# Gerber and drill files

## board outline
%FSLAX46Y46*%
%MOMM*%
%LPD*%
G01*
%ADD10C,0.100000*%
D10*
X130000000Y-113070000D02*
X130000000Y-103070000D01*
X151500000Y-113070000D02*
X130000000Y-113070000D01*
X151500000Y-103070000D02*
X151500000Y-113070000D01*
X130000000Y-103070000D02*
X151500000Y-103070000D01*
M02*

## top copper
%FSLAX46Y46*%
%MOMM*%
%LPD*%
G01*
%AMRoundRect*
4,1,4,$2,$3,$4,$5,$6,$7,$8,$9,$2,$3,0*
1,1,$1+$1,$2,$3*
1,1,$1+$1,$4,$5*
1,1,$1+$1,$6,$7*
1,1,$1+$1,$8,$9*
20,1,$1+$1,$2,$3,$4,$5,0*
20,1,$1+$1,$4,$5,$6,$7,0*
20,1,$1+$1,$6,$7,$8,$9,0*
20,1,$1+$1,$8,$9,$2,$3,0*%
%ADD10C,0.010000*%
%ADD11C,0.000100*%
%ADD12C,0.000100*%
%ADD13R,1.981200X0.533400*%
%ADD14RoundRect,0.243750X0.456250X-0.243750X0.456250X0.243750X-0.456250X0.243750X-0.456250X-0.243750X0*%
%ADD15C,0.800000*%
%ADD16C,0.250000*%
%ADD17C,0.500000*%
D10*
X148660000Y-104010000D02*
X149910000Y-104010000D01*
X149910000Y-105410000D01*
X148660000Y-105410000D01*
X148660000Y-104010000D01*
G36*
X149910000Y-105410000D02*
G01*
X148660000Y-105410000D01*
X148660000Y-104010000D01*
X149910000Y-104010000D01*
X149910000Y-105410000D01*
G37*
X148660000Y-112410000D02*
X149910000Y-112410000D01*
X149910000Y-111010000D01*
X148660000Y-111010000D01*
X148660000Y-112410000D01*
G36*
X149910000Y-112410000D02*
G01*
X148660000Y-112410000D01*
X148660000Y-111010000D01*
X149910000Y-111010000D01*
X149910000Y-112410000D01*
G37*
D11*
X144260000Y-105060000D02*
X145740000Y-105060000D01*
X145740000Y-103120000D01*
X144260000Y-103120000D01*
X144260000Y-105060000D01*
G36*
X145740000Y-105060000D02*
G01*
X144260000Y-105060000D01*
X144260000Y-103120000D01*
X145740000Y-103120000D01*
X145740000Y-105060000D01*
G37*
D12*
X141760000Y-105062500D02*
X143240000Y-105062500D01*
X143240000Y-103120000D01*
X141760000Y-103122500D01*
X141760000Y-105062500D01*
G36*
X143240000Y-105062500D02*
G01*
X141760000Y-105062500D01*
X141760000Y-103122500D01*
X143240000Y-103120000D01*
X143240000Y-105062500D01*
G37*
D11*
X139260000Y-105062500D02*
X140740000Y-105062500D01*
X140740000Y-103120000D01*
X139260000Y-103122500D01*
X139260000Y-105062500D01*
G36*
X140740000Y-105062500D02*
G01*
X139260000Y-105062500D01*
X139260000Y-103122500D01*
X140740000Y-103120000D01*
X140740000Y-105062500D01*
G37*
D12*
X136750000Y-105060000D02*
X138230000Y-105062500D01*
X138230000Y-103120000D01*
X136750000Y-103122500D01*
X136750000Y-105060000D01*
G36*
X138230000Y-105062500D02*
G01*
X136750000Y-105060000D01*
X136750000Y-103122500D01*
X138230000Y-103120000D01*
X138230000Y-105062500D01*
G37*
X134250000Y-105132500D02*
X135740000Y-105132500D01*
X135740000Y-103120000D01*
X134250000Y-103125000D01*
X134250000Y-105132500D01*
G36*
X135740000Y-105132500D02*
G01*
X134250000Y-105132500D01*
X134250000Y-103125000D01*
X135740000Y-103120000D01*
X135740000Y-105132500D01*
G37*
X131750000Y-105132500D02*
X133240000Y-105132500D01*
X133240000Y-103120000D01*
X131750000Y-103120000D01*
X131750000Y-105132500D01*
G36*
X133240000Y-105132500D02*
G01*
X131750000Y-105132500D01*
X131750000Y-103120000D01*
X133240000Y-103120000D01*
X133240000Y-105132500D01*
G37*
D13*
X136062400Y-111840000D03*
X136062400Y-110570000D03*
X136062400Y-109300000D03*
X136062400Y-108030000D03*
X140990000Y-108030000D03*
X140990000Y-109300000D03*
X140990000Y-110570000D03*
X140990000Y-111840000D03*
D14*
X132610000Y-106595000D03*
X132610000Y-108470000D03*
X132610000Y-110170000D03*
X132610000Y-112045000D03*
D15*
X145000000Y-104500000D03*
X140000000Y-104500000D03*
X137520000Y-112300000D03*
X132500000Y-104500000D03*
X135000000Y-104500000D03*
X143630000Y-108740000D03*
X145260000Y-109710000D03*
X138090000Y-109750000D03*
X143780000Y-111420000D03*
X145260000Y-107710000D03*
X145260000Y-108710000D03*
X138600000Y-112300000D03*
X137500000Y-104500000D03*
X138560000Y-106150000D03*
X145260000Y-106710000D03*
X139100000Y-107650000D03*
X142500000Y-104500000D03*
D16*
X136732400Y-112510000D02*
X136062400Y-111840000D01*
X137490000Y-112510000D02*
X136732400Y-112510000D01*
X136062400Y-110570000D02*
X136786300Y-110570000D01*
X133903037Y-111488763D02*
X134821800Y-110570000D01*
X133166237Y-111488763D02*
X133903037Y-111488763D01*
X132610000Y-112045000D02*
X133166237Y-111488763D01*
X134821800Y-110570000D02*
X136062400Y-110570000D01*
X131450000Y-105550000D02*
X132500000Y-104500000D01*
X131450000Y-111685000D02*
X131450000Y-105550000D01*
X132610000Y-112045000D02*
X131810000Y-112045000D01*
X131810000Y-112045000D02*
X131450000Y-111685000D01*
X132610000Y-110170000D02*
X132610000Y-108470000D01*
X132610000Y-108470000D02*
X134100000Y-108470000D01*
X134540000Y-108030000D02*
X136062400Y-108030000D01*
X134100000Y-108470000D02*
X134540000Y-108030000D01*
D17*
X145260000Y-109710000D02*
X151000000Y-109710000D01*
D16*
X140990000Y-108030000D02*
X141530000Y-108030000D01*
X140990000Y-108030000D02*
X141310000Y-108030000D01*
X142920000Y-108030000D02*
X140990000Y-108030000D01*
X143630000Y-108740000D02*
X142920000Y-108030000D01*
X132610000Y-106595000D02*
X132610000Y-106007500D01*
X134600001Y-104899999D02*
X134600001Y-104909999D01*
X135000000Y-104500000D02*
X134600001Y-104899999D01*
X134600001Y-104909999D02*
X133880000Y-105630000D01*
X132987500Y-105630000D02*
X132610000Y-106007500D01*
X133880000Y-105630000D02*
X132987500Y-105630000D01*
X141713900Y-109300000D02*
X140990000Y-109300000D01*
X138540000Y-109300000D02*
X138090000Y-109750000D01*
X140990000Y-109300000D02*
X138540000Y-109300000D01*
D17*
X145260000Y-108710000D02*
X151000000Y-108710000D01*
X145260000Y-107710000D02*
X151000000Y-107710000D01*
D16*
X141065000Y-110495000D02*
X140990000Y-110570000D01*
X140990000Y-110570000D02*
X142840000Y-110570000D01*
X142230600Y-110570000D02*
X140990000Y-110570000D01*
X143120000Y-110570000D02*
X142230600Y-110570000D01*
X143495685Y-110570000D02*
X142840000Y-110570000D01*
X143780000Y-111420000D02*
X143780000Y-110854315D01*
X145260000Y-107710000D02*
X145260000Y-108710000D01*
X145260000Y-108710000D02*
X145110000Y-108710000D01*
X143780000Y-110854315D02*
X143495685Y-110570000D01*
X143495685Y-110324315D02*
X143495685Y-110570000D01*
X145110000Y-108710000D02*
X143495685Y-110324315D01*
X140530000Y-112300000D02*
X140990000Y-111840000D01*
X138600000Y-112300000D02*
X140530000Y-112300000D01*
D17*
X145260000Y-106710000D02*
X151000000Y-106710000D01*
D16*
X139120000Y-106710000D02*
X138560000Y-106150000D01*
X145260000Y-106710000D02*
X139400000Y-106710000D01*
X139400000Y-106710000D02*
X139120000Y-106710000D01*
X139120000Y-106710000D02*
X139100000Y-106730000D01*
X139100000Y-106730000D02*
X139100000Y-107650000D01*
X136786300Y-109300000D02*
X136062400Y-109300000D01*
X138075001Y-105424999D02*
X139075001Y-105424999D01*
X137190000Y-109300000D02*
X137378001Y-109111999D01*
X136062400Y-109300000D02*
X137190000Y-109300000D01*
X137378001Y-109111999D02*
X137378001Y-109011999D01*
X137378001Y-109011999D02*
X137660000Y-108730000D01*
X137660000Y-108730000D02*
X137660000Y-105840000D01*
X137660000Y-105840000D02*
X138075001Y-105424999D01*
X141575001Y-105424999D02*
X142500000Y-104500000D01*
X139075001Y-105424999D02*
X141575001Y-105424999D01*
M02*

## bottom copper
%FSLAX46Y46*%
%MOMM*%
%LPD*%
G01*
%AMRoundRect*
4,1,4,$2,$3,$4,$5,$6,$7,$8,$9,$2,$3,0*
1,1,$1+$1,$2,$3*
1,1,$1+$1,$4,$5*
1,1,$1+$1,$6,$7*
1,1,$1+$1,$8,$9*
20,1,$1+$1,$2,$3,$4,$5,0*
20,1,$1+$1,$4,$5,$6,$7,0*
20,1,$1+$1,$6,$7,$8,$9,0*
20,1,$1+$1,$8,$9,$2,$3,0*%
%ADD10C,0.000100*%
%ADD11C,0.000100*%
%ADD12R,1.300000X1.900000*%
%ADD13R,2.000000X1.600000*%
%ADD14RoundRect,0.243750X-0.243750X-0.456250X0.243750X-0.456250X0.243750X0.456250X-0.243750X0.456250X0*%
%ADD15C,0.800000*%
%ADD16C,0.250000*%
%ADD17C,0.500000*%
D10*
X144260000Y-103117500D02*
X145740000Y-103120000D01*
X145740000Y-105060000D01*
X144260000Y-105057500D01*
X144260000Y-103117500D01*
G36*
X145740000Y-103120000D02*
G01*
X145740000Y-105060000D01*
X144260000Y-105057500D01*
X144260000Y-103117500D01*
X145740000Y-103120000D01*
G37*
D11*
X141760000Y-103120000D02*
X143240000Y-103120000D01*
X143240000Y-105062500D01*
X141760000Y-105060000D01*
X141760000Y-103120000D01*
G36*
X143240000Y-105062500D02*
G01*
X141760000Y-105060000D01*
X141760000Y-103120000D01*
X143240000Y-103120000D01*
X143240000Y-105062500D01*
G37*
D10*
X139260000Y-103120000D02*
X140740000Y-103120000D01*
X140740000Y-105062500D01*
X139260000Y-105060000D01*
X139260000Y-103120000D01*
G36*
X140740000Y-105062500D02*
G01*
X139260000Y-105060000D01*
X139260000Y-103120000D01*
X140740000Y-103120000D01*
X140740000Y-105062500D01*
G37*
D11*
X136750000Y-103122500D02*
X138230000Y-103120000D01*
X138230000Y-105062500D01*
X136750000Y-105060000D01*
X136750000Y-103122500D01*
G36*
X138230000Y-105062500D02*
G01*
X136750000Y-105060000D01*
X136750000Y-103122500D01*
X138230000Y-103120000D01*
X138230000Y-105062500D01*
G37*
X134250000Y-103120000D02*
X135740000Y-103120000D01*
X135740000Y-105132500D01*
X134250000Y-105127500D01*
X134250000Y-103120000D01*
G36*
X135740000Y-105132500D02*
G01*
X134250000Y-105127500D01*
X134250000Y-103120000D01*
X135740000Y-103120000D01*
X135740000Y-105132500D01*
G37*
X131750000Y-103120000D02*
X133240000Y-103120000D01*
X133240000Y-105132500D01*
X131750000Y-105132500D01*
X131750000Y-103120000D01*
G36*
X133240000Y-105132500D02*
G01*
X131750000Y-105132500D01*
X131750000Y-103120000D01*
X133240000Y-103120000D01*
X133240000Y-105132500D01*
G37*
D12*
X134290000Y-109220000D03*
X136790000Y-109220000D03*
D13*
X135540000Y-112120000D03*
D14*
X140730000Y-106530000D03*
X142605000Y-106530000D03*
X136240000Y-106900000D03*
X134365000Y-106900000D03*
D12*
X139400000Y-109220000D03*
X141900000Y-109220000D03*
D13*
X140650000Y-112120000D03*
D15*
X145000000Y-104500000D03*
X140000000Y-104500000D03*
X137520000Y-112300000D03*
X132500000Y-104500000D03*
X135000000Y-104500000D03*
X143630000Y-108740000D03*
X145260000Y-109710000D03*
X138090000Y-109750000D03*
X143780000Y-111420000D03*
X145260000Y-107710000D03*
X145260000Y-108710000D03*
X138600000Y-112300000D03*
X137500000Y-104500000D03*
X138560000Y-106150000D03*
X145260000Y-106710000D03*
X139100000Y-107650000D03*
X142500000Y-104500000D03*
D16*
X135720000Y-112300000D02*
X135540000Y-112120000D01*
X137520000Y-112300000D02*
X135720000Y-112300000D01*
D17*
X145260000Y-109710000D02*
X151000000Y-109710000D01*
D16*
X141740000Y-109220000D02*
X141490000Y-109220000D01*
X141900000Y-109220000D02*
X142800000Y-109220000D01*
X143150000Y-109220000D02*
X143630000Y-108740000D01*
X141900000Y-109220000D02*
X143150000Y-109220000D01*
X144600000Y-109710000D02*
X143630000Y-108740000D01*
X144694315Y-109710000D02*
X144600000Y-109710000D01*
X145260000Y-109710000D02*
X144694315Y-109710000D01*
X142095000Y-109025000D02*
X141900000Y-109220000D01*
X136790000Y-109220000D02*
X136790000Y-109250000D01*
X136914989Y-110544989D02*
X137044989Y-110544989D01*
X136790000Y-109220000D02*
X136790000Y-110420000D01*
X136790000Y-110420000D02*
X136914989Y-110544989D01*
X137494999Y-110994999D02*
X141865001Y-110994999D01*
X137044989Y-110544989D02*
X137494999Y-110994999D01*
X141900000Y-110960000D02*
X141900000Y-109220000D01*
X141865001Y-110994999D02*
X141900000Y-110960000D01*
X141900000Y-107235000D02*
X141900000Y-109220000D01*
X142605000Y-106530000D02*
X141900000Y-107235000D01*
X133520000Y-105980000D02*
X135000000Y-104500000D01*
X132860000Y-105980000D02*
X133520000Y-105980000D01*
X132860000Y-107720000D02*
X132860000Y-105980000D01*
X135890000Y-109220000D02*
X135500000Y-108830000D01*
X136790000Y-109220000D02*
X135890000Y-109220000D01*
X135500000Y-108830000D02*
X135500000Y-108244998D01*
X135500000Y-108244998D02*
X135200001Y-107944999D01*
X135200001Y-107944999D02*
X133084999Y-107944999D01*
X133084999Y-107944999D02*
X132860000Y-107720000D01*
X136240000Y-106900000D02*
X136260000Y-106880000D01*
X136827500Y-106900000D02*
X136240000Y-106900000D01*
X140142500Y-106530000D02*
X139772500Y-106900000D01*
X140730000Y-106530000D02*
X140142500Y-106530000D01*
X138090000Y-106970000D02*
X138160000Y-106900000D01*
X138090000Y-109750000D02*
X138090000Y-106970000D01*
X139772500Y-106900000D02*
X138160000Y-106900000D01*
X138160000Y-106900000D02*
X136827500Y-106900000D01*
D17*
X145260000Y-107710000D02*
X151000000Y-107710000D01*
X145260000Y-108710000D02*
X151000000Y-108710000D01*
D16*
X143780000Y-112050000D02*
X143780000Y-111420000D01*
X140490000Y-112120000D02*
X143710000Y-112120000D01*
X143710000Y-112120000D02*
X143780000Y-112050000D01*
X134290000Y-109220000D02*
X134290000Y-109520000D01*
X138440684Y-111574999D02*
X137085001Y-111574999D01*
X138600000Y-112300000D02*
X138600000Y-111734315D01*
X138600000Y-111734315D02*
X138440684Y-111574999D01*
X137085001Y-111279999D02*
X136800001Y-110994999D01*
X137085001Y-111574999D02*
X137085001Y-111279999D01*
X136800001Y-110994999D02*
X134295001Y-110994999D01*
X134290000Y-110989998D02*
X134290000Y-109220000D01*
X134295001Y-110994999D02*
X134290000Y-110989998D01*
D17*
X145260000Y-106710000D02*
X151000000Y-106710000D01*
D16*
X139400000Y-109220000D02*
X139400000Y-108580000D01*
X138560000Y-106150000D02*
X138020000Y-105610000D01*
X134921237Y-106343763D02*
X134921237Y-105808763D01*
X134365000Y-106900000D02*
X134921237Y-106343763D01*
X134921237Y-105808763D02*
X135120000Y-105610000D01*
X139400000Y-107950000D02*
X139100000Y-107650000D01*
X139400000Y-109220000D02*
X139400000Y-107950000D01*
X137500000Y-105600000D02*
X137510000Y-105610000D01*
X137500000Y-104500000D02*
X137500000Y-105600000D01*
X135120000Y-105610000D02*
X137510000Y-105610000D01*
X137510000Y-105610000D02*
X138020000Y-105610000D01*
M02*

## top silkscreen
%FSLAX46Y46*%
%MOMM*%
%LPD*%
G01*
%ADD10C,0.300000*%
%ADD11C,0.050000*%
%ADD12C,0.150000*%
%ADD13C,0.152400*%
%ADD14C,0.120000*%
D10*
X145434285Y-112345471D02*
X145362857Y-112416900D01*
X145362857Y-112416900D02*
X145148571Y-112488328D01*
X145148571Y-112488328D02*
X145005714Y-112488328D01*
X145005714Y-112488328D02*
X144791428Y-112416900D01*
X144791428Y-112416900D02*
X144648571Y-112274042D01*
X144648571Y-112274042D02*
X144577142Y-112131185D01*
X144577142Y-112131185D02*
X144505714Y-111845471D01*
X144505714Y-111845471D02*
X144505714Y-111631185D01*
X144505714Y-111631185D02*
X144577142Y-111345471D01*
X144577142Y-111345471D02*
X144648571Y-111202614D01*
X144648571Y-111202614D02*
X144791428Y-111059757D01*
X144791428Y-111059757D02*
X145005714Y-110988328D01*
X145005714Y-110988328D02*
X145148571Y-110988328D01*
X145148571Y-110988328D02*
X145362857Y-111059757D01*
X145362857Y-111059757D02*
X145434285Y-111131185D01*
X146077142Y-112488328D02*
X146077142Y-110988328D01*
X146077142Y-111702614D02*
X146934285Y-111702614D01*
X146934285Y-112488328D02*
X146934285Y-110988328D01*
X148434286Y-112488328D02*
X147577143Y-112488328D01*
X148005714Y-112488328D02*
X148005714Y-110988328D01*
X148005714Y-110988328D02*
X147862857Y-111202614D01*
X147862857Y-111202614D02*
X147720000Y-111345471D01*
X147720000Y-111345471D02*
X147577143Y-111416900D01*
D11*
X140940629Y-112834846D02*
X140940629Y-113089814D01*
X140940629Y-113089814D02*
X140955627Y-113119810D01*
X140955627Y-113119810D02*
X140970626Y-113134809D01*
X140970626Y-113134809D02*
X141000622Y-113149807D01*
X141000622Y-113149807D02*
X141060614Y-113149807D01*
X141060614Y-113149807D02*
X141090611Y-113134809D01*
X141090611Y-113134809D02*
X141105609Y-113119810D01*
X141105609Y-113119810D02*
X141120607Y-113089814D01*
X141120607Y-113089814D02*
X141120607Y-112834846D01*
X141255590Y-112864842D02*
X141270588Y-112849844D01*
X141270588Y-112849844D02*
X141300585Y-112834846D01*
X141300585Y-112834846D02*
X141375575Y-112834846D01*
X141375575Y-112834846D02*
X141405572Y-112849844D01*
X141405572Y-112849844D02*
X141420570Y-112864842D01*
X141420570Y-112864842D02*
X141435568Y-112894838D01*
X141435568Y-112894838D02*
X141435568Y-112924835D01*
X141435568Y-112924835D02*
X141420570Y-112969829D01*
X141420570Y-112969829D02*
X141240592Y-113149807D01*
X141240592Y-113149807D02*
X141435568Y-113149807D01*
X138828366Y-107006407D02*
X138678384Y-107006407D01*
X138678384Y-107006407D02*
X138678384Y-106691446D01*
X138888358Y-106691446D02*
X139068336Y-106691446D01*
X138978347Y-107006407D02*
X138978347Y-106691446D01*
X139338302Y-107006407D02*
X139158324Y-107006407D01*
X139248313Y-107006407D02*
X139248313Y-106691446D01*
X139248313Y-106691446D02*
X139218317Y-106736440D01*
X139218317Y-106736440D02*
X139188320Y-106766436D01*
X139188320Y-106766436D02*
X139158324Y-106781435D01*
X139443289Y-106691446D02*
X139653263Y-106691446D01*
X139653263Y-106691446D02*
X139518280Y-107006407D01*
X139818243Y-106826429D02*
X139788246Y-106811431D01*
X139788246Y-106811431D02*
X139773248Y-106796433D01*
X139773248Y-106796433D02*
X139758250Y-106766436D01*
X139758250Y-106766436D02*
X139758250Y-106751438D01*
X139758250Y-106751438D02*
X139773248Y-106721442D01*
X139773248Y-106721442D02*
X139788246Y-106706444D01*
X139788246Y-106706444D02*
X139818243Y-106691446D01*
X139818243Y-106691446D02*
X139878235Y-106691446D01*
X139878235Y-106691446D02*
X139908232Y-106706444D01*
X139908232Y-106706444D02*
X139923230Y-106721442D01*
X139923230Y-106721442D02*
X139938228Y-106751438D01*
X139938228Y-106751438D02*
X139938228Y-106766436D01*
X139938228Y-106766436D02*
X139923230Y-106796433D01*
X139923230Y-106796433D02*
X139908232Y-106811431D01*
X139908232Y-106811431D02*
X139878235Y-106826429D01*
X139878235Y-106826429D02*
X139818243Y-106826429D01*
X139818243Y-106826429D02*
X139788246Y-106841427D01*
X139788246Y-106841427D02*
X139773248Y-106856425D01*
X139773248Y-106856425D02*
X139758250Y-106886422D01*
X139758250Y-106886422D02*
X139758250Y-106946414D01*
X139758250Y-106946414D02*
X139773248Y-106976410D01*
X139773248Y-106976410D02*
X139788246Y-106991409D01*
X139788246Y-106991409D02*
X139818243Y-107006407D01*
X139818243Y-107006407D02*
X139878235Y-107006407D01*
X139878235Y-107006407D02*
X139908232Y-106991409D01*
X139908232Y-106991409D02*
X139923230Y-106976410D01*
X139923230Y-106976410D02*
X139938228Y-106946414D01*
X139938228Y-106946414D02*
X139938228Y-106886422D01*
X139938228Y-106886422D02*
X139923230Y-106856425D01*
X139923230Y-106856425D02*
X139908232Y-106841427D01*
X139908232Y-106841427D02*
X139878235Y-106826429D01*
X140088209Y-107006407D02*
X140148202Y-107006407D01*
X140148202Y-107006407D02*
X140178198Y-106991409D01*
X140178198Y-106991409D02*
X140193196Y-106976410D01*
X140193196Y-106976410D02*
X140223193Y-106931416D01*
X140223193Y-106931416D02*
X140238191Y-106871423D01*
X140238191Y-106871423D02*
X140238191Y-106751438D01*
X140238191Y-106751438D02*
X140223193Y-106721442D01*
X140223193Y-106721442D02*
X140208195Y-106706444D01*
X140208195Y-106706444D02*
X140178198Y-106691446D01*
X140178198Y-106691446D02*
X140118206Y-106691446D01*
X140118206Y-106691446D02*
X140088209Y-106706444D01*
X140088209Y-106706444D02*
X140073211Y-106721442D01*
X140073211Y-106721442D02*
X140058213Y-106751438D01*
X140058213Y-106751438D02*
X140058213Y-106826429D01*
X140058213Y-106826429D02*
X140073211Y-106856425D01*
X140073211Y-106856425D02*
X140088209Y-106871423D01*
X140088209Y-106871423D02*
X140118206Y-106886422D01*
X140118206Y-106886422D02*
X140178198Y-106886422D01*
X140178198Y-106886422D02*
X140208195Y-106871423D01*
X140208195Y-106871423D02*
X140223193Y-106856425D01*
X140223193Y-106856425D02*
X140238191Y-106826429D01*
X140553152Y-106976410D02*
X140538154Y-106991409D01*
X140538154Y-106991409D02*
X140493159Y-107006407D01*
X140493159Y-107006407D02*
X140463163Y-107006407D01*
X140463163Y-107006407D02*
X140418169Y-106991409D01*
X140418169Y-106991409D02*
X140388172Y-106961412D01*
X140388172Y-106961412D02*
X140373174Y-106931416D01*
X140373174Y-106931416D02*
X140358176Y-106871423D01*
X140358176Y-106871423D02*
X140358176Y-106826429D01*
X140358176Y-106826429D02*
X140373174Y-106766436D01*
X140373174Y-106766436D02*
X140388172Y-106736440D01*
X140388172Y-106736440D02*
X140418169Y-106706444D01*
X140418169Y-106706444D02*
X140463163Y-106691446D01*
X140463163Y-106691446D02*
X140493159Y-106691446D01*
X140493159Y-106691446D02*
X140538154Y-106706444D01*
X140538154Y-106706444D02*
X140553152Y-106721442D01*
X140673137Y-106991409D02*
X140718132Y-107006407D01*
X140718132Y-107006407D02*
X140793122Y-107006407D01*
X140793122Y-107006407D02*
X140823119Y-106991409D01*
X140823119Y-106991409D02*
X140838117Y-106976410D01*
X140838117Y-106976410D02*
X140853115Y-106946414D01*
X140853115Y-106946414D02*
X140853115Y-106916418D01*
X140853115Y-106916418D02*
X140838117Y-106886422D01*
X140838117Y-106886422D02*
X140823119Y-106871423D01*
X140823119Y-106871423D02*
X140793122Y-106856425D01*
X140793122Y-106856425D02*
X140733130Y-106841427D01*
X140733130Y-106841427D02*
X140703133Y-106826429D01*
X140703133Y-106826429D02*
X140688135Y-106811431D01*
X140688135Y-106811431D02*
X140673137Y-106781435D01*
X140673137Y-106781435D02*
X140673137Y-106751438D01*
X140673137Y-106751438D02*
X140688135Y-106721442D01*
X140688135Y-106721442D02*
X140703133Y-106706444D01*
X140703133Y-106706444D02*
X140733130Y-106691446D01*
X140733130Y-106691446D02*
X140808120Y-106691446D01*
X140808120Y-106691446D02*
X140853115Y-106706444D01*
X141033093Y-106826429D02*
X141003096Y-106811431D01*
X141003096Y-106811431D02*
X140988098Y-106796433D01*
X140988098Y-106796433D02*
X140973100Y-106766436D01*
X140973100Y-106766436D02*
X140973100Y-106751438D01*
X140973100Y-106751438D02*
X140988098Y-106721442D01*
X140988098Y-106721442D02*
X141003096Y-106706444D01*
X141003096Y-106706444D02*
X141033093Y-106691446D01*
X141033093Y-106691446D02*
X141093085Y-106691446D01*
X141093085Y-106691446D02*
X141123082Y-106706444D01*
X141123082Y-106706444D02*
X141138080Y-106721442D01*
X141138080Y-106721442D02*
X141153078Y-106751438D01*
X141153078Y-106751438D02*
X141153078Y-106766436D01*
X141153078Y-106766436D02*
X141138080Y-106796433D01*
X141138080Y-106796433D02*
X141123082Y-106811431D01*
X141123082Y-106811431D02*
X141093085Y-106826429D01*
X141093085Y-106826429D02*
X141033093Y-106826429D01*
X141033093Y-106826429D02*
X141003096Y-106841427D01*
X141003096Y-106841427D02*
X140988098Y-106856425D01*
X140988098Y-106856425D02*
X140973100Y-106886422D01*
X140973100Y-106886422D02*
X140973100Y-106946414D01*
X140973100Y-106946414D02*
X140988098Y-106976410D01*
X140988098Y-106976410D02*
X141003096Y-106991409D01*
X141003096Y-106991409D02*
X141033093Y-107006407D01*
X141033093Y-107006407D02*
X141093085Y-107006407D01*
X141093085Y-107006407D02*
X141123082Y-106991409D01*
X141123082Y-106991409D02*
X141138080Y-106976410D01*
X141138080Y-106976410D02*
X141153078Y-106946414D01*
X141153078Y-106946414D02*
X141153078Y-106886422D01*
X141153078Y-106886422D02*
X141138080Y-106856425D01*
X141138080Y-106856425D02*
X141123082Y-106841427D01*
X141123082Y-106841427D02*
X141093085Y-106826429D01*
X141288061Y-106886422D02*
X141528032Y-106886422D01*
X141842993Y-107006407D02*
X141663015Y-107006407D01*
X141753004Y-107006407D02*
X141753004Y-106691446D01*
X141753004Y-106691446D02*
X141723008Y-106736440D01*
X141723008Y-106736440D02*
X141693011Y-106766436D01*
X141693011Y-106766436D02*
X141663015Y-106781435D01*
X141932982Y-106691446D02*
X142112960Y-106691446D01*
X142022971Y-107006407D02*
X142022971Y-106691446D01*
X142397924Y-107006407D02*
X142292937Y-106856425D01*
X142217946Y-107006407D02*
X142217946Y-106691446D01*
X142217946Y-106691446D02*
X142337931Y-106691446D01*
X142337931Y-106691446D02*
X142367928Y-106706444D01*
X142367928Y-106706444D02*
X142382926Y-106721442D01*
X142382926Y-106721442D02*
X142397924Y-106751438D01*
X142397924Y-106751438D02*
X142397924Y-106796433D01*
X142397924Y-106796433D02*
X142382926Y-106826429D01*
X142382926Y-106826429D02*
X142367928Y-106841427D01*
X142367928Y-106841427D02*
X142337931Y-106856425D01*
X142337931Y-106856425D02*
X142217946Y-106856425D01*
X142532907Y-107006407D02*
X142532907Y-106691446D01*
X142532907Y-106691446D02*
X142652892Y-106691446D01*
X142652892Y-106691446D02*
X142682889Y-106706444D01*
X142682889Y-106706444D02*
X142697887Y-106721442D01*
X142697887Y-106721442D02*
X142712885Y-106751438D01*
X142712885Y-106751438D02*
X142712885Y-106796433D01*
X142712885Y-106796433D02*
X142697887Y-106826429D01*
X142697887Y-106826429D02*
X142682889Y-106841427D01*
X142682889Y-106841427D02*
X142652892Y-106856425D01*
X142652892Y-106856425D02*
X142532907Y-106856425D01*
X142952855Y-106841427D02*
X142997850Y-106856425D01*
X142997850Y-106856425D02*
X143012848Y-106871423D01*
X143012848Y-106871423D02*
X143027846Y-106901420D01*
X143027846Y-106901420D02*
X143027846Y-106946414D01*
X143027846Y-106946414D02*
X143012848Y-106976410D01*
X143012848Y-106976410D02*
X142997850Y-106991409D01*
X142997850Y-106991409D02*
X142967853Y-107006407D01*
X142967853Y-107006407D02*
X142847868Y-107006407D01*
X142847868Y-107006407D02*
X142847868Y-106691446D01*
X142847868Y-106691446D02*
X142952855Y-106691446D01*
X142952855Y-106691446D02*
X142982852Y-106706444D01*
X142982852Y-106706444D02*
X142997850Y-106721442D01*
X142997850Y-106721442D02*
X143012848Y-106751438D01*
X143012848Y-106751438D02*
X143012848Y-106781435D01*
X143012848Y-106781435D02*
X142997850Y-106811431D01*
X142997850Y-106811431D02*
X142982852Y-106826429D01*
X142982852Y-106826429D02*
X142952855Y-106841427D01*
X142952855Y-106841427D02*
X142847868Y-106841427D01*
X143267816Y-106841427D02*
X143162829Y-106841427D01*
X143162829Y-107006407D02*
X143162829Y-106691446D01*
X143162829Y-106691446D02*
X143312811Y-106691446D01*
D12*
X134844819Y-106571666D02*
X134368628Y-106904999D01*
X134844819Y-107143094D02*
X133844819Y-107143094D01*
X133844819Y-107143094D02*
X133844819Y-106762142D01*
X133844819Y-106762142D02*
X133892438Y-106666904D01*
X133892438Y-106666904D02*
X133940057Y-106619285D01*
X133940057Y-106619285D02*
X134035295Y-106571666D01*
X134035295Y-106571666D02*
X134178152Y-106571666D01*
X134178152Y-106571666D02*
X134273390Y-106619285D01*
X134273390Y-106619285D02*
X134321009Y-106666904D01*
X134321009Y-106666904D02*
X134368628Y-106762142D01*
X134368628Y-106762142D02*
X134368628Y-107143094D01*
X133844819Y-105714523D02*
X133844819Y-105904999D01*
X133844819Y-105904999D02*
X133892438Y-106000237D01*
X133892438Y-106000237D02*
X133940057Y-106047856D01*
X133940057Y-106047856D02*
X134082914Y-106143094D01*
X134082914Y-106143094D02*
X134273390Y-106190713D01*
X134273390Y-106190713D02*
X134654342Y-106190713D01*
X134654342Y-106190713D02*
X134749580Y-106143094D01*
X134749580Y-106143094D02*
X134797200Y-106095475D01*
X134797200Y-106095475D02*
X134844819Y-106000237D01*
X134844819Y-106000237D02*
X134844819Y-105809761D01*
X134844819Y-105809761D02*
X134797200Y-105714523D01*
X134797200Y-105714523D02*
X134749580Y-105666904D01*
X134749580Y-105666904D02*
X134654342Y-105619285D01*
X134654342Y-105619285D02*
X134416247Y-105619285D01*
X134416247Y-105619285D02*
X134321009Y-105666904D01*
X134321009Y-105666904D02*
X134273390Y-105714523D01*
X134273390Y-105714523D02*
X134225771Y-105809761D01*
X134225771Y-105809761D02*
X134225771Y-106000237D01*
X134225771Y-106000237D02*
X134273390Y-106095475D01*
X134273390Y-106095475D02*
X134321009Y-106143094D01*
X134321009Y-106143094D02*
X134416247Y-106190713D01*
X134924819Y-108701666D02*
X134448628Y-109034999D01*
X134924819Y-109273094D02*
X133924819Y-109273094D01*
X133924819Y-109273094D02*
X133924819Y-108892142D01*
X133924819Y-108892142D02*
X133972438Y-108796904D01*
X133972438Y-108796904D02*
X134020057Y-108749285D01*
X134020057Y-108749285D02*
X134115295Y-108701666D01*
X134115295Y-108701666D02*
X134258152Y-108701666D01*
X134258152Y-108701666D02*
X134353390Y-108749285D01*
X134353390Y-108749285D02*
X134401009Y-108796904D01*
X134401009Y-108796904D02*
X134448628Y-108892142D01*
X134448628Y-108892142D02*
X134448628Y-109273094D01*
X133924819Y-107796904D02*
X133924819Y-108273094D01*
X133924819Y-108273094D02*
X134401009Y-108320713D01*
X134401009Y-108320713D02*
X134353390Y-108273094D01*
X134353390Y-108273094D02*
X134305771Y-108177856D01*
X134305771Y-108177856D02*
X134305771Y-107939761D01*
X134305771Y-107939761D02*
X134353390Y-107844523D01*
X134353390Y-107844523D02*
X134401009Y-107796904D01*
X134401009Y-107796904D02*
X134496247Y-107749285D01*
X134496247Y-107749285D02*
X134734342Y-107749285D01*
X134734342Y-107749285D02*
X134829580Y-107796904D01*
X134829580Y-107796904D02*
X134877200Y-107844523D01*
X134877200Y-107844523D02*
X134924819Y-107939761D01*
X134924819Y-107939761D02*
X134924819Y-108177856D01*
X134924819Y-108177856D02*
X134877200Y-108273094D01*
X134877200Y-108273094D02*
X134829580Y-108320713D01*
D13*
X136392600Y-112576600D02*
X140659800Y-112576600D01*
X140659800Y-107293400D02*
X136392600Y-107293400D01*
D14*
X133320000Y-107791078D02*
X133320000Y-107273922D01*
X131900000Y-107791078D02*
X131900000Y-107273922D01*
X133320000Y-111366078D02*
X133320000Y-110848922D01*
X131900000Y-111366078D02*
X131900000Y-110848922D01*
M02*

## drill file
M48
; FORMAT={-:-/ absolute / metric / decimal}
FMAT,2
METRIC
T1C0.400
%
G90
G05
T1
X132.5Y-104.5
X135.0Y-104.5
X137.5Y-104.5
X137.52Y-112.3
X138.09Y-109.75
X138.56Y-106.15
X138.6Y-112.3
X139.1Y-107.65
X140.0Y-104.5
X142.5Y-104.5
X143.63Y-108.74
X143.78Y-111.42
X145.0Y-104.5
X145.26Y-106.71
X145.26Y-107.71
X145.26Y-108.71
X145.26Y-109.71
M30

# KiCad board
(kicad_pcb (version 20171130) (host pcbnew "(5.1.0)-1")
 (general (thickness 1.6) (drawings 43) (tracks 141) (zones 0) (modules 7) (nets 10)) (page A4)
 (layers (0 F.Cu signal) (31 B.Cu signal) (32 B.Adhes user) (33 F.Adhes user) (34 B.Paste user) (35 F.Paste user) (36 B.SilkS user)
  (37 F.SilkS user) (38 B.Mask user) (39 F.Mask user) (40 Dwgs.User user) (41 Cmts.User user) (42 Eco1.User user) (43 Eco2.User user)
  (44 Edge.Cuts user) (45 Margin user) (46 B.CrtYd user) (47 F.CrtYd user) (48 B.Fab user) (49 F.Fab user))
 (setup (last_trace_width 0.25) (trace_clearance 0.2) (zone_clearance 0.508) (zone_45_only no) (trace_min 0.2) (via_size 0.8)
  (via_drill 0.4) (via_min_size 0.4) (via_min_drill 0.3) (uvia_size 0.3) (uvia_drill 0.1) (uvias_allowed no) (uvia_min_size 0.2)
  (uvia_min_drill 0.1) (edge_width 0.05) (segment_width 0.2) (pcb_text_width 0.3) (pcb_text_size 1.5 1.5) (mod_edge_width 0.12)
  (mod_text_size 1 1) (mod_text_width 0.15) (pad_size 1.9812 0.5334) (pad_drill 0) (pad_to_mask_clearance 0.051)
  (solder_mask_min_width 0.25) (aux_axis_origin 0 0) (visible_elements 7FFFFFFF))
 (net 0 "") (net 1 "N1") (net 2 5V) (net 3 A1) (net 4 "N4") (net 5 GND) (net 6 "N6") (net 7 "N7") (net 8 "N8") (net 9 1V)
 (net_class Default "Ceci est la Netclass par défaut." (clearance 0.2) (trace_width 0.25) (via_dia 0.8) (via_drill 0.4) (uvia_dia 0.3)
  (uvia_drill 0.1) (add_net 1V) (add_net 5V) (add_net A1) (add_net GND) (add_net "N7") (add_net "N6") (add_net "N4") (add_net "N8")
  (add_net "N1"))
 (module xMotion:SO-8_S (layer F.Cu) (at 138.5262 109.935 180)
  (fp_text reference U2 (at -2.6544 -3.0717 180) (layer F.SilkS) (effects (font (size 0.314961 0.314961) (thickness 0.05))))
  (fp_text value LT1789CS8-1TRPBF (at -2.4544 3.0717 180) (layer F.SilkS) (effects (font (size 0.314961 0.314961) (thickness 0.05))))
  (fp_line (start 2.1336 -2.6416) (end -2.1336 -2.6416) (layer F.SilkS) (width 0.1524))
  (fp_line (start -2.1336 2.6416) (end 2.1336 2.6416) (layer F.SilkS) (width 0.1524))
  (pad 8 smd rect (at 2.4638 -1.905 180) (size 1.9812 0.5334) (layers F.Cu F.Paste F.Mask) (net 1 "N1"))
  (pad 7 smd rect (at 2.4638 -0.635 180) (size 1.9812 0.5334) (layers F.Cu F.Paste F.Mask) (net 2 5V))
  (pad 6 smd rect (at 2.4638 0.635 180) (size 1.9812 0.5334) (layers F.Cu F.Paste F.Mask) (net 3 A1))
  (pad 5 smd rect (at 2.4638 1.905 180) (size 1.9812 0.5334) (layers F.Cu F.Paste F.Mask) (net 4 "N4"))
  (pad 4 smd rect (at -2.4638 1.905 180) (size 1.9812 0.5334) (layers F.Cu F.Paste F.Mask) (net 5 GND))
  (pad 3 smd rect (at -2.4638 0.635 180) (size 1.9812 0.5334) (layers F.Cu F.Paste F.Mask) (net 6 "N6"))
  (pad 2 smd rect (at -2.4638 -0.635 180) (size 1.9812 0.5334) (layers F.Cu F.Paste F.Mask) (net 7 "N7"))
  (pad 1 smd rect (at -2.4638 -1.905 180) (size 1.9812 0.5334) (layers F.Cu F.Paste F.Mask) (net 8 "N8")))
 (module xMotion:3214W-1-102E (layer B.Cu) (at 135.54 112.12 90)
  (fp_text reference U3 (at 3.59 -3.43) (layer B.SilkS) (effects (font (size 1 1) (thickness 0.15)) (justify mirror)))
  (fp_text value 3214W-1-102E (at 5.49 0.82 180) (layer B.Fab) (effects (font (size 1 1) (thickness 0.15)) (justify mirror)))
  (pad 3 smd rect (at 2.9 -1.25 90) (size 1.9 1.3) (layers B.Cu B.Paste B.Mask) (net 8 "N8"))
  (pad 2 smd rect (at 2.9 1.25 90) (size 1.9 1.3) (layers B.Cu B.Paste B.Mask) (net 5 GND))
  (pad 1 smd rect (at 0 0 90) (size 1.6 2) (layers B.Cu B.Paste B.Mask) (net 1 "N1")))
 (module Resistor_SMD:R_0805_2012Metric (layer F.Cu) (at 132.61 107.5325 90)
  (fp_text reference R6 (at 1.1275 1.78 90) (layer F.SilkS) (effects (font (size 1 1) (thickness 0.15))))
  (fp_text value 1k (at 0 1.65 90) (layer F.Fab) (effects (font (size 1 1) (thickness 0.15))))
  (fp_line (start -0.258578 0.71) (end 0.258578 0.71) (layer F.SilkS) (width 0.12))
  (fp_line (start -0.258578 -0.71) (end 0.258578 -0.71) (layer F.SilkS) (width 0.12))
  (pad 2 smd roundrect (at 0.9375 0 90) (size 0.975 1.4) (layers F.Cu F.Paste F.Mask) (roundrect_rratio 0.25) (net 5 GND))
  (pad 1 smd roundrect (at -0.9375 0 90) (size 0.975 1.4) (layers F.Cu F.Paste F.Mask) (roundrect_rratio 0.25) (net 4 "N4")))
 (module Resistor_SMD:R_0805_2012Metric (layer F.Cu) (at 132.61 111.1075 90)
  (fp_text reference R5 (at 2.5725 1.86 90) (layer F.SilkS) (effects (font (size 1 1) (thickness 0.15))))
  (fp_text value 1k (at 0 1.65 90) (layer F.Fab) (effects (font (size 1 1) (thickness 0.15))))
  (fp_line (start -0.258578 0.71) (end 0.258578 0.71) (layer F.SilkS) (width 0.12))
  (fp_line (start -0.258578 -0.71) (end 0.258578 -0.71) (layer F.SilkS) (width 0.12))
  (pad 2 smd roundrect (at 0.9375 0 90) (size 0.975 1.4) (layers F.Cu F.Paste F.Mask) (roundrect_rratio 0.25) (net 4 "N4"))
  (pad 1 smd roundrect (at -0.9375 0 90) (size 0.975 1.4) (layers F.Cu F.Paste F.Mask) (roundrect_rratio 0.25) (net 2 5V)))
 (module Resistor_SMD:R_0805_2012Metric (layer B.Cu) (at 141.6675 106.53)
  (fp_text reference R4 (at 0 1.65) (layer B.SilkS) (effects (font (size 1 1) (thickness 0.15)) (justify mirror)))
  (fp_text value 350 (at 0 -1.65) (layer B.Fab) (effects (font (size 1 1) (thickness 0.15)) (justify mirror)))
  (pad 1 smd roundrect (at -0.9375 0) (size 0.975 1.4) (layers B.Cu B.Paste B.Mask) (roundrect_rratio 0.25) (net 6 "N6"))
  (pad 2 smd roundrect (at 0.9375 0) (size 0.975 1.4) (layers B.Cu B.Paste B.Mask) (roundrect_rratio 0.25) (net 5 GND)))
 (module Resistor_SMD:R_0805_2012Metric (layer B.Cu) (at 135.3025 106.9)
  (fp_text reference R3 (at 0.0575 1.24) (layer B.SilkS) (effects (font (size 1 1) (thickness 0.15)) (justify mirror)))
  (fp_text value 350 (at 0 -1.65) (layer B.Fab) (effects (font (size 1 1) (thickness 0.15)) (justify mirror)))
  (pad 2 smd roundrect (at 0.9375 0) (size 0.975 1.4) (layers B.Cu B.Paste B.Mask) (roundrect_rratio 0.25) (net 6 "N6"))
  (pad 1 smd roundrect (at -0.9375 0) (size 0.975 1.4) (layers B.Cu B.Paste B.Mask) (roundrect_rratio 0.25) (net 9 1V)))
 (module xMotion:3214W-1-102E (layer B.Cu) (at 140.65 112.12 90)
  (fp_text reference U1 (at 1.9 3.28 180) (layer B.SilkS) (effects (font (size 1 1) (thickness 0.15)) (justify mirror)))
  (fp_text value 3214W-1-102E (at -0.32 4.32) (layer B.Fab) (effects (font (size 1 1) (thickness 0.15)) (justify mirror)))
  (pad 3 smd rect (at 2.9 -1.25 90) (size 1.9 1.3) (layers B.Cu B.Paste B.Mask) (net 9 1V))
  (pad 2 smd rect (at 2.9 1.25 90) (size 1.9 1.3) (layers B.Cu B.Paste B.Mask) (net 5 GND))
  (pad 1 smd rect (at 0 0 90) (size 1.6 2) (layers B.Cu B.Paste B.Mask) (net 7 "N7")))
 (gr_poly (pts (xy 148.66 104.01) (xy 149.91 104.01) (xy 149.91 105.41) (xy 148.66 105.41)) (layer F.Cu) (width 0.01))
 (gr_poly (pts (xy 148.66 112.41) (xy 149.91 112.41) (xy 149.91 111.01) (xy 148.66 111.01)) (layer F.Cu) (width 0.01))
 (gr_poly (pts (xy 144.26 103.1175) (xy 145.74 103.12) (xy 145.74 105.06) (xy 144.26 105.0575)) (layer B.Cu) (width 0.0001))
 (gr_poly (pts (xy 144.26 105.06) (xy 145.74 105.06) (xy 145.74 103.12) (xy 144.26 103.12)) (layer F.Cu) (width 0.0001))
 (gr_poly (pts (xy 141.76 103.12) (xy 143.24 103.12) (xy 143.24 105.0625) (xy 141.76 105.06)) (layer B.Cu) (width 0.0001))
 (gr_poly (pts (xy 141.76 105.0625) (xy 143.24 105.0625) (xy 143.24 103.12) (xy 141.76 103.1225)) (layer F.Cu) (width 0.0001))
 (gr_poly (pts (xy 139.26 103.12) (xy 140.74 103.12) (xy 140.74 105.0625) (xy 139.26 105.06)) (layer B.Cu) (width 0.0001))
 (gr_poly (pts (xy 139.26 105.0625) (xy 140.74 105.0625) (xy 140.74 103.12) (xy 139.26 103.1225)) (layer F.Cu) (width 0.0001))
 (gr_poly (pts (xy 136.75 103.1225) (xy 138.23 103.12) (xy 138.23 105.0625) (xy 136.75 105.06)) (layer B.Cu) (width 0.0001))
 (gr_poly (pts (xy 136.75 105.06) (xy 138.23 105.0625) (xy 138.23 103.12) (xy 136.75 103.1225)) (layer F.Cu) (width 0.0001))
 (gr_poly (pts (xy 134.25 103.12) (xy 135.74 103.12) (xy 135.74 105.1325) (xy 134.25 105.1275)) (layer B.Cu) (width 0.0001))
 (gr_poly (pts (xy 134.25 105.1325) (xy 135.74 105.1325) (xy 135.74 103.12) (xy 134.25 103.125)) (layer F.Cu) (width 0.0001))
 (gr_poly (pts (xy 131.75 103.12) (xy 133.24 103.12) (xy 133.24 105.1325) (xy 131.75 105.1325)) (layer B.Cu) (width 0.0001))
 (gr_poly (pts (xy 131.75 105.1325) (xy 133.24 105.1325) (xy 133.24 103.12) (xy 131.75 103.12)) (layer F.Cu) (width 0.0001))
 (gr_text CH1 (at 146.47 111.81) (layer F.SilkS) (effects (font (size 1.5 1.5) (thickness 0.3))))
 (gr_line (start 130 113.07) (end 130 103.07) (layer Edge.Cuts) (width 0.1))
 (gr_line (start 151.5 113.07) (end 130 113.07) (layer Edge.Cuts) (width 0.1))
 (gr_line (start 151.5 103.07) (end 151.5 113.07) (layer Edge.Cuts) (width 0.1))
 (gr_line (start 130 103.07) (end 151.5 103.07) (layer Edge.Cuts) (width 0.1))
 (via (at 145 104.5) (size 0.8) (drill 0.4) (layers F.Cu B.Cu) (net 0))
 (via (at 140 104.5) (size 0.8) (drill 0.4) (layers F.Cu B.Cu) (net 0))
 (via (at 137.52 112.3) (size 0.8) (drill 0.4) (layers F.Cu B.Cu) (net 1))
 (segment (start 136.7324 112.51) (end 136.0624 111.84) (width 0.25) (layer F.Cu) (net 1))
 (segment (start 137.49 112.51) (end 136.7324 112.51) (width 0.25) (layer F.Cu) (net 1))
 (segment (start 135.72 112.3) (end 135.54 112.12) (width 0.25) (layer B.Cu) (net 1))
 (segment (start 137.52 112.3) (end 135.72 112.3) (width 0.25) (layer B.Cu) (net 1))
 (via (at 132.5 104.5) (size 0.8) (drill 0.4) (layers F.Cu B.Cu) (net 2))
 (segment (start 136.0624 110.57) (end 136.7863 110.57) (width 0.25) (layer F.Cu) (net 2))
 (segment (start 133.903037 111.488763) (end 134.8218 110.57) (width 0.25) (layer F.Cu) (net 2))
 (segment (start 133.166237 111.488763) (end 133.903037 111.488763) (width 0.25) (layer F.Cu) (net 2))
 (segment (start 132.61 112.045) (end 133.166237 111.488763) (width 0.25) (layer F.Cu) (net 2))
 (segment (start 134.8218 110.57) (end 136.0624 110.57) (width 0.25) (layer F.Cu) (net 2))
 (segment (start 131.45 105.55) (end 132.5 104.5) (width 0.25) (layer F.Cu) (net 2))
 (segment (start 131.45 111.685) (end 131.45 105.55) (width 0.25) (layer F.Cu) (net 2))
 (segment (start 132.61 112.045) (end 131.81 112.045) (width 0.25) (layer F.Cu) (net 2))
 (segment (start 131.81 112.045) (end 131.45 111.685) (width 0.25) (layer F.Cu) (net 2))
 (segment (start 132.61 110.17) (end 132.61 108.47) (width 0.25) (layer F.Cu) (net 4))
 (segment (start 132.61 108.47) (end 134.1 108.47) (width 0.25) (layer F.Cu) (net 4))
 (segment (start 134.54 108.03) (end 136.0624 108.03) (width 0.25) (layer F.Cu) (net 4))
 (segment (start 134.1 108.47) (end 134.54 108.03) (width 0.25) (layer F.Cu) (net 4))
 (via (at 135 104.5) (size 0.8) (drill 0.4) (layers F.Cu B.Cu) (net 5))
 (via (at 143.63 108.74) (size 0.8) (drill 0.4) (layers F.Cu B.Cu) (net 5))
 (segment (start 145.26 109.71) (end 151 109.71) (width 0.5) (layer F.Cu) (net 5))
 (segment (start 140.99 108.03) (end 141.53 108.03) (width 0.25) (layer F.Cu) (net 5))
 (segment (start 140.99 108.03) (end 141.31 108.03) (width 0.25) (layer F.Cu) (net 5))
 (segment (start 145.26 109.71) (end 151 109.71) (width 0.5) (layer B.Cu) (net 5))
 (via (at 145.26 109.71) (size 0.8) (drill 0.4) (layers F.Cu B.Cu) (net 5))
 (segment (start 141.74 109.22) (end 141.49 109.22) (width 0.25) (layer B.Cu) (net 5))
 (segment (start 141.9 109.22) (end 142.8 109.22) (width 0.25) (layer B.Cu) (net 5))
 (segment (start 142.92 108.03) (end 140.99 108.03) (width 0.25) (layer F.Cu) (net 5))
 (segment (start 143.63 108.74) (end 142.92 108.03) (width 0.25) (layer F.Cu) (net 5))
 (segment (start 143.15 109.22) (end 143.63 108.74) (width 0.25) (layer B.Cu) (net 5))
 (segment (start 141.9 109.22) (end 143.15 109.22) (width 0.25) (layer B.Cu) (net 5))
 (segment (start 144.6 109.71) (end 143.63 108.74) (width 0.25) (layer B.Cu) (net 5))
 (segment (start 144.694315 109.71) (end 144.6 109.71) (width 0.25) (layer B.Cu) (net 5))
 (segment (start 145.26 109.71) (end 144.694315 109.71) (width 0.25) (layer B.Cu) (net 5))
 (segment (start 142.095 109.025) (end 141.9 109.22) (width 0.25) (layer B.Cu) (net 5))
 (segment (start 136.79 109.22) (end 136.79 109.25) (width 0.25) (layer B.Cu) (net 5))
 (segment (start 136.914989 110.544989) (end 137.044989 110.544989) (width 0.25) (layer B.Cu) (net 5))
 (segment (start 136.79 109.22) (end 136.79 110.42) (width 0.25) (layer B.Cu) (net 5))
 (segment (start 136.79 110.42) (end 136.914989 110.544989) (width 0.25) (layer B.Cu) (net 5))
 (segment (start 137.494999 110.994999) (end 141.865001 110.994999) (width 0.25) (layer B.Cu) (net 5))
 (segment (start 137.044989 110.544989) (end 137.494999 110.994999) (width 0.25) (layer B.Cu) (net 5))
 (segment (start 141.9 110.96) (end 141.9 109.22) (width 0.25) (layer B.Cu) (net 5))
 (segment (start 141.865001 110.994999) (end 141.9 110.96) (width 0.25) (layer B.Cu) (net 5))
 (segment (start 141.9 107.235) (end 141.9 109.22) (width 0.25) (layer B.Cu) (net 5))
 (segment (start 142.605 106.53) (end 141.9 107.235) (width 0.25) (layer B.Cu) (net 5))
 (segment (start 132.61 106.595) (end 132.61 106.0075) (width 0.25) (layer F.Cu) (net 5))
 (segment (start 134.600001 104.899999) (end 134.600001 104.909999) (width 0.25) (layer F.Cu) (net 5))
 (segment (start 135 104.5) (end 134.600001 104.899999) (width 0.25) (layer F.Cu) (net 5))
 (segment (start 134.600001 104.909999) (end 133.88 105.63) (width 0.25) (layer F.Cu) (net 5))
 (segment (start 132.9875 105.63) (end 132.61 106.0075) (width 0.25) (layer F.Cu) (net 5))
 (segment (start 133.88 105.63) (end 132.9875 105.63) (width 0.25) (layer F.Cu) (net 5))
 (segment (start 133.52 105.98) (end 135 104.5) (width 0.25) (layer B.Cu) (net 5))
 (segment (start 132.86 105.98) (end 133.52 105.98) (width 0.25) (layer B.Cu) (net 5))
 (segment (start 132.86 107.72) (end 132.86 105.98) (width 0.25) (layer B.Cu) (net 5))
 (segment (start 135.89 109.22) (end 135.5 108.83) (width 0.25) (layer B.Cu) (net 5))
 (segment (start 136.79 109.22) (end 135.89 109.22) (width 0.25) (layer B.Cu) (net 5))
 (segment (start 135.5 108.83) (end 135.5 108.244998) (width 0.25) (layer B.Cu) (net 5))
 (segment (start 135.5 108.244998) (end 135.200001 107.944999) (width 0.25) (layer B.Cu) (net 5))
 (segment (start 135.200001 107.944999) (end 133.084999 107.944999) (width 0.25) (layer B.Cu) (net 5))
 (segment (start 133.084999 107.944999) (end 132.86 107.72) (width 0.25) (layer B.Cu) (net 5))
 (via (at 138.09 109.75) (size 0.8) (drill 0.4) (layers F.Cu B.Cu) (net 6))
 (segment (start 141.7139 109.3) (end 140.99 109.3) (width 0.25) (layer F.Cu) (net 6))
 (segment (start 136.24 106.9) (end 136.26 106.88) (width 0.25) (layer B.Cu) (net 6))
 (segment (start 136.8275 106.9) (end 136.24 106.9) (width 0.25) (layer B.Cu) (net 6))
 (segment (start 140.1425 106.53) (end 139.7725 106.9) (width 0.25) (layer B.Cu) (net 6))
 (segment (start 140.73 106.53) (end 140.1425 106.53) (width 0.25) (layer B.Cu) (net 6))
 (segment (start 138.54 109.3) (end 138.09 109.75) (width 0.25) (layer F.Cu) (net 6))
 (segment (start 140.99 109.3) (end 138.54 109.3) (width 0.25) (layer F.Cu) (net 6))
 (segment (start 138.09 106.97) (end 138.16 106.9) (width 0.25) (layer B.Cu) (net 6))
 (segment (start 138.09 109.75) (end 138.09 106.97) (width 0.25) (layer B.Cu) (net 6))
 (segment (start 139.7725 106.9) (end 138.16 106.9) (width 0.25) (layer B.Cu) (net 6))
 (segment (start 138.16 106.9) (end 136.8275 106.9) (width 0.25) (layer B.Cu) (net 6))
 (via (at 143.78 111.42) (size 0.8) (drill 0.4) (layers F.Cu B.Cu) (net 7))
 (segment (start 145.26 108.71) (end 151 108.71) (width 0.5) (layer F.Cu) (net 7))
 (segment (start 145.26 107.71) (end 151 107.71) (width 0.5) (layer F.Cu) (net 7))
 (segment (start 145.26 107.71) (end 151 107.71) (width 0.5) (layer B.Cu) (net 7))
 (segment (start 145.26 108.71) (end 151 108.71) (width 0.5) (layer B.Cu) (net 7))
 (via (at 145.26 107.71) (size 0.8) (drill 0.4) (layers F.Cu B.Cu) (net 7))
 (via (at 145.26 108.71) (size 0.8) (drill 0.4) (layers F.Cu B.Cu) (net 7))
 (segment (start 141.065 110.495) (end 140.99 110.57) (width 0.25) (layer F.Cu) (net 7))
 (segment (start 140.99 110.57) (end 142.84 110.57) (width 0.25) (layer F.Cu) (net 7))
 (segment (start 142.2306 110.57) (end 140.99 110.57) (width 0.25) (layer F.Cu) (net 7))
 (segment (start 143.12 110.57) (end 142.2306 110.57) (width 0.25) (layer F.Cu) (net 7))
 (segment (start 143.495685 110.57) (end 142.84 110.57) (width 0.25) (layer F.Cu) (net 7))
 (segment (start 143.78 111.42) (end 143.78 110.854315) (width 0.25) (layer F.Cu) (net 7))
 (segment (start 143.78 112.05) (end 143.78 111.42) (width 0.25) (layer B.Cu) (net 7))
 (segment (start 140.49 112.12) (end 143.71 112.12) (width 0.25) (layer B.Cu) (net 7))
 (segment (start 143.71 112.12) (end 143.78 112.05) (width 0.25) (layer B.Cu) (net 7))
 (segment (start 145.26 107.71) (end 145.26 108.71) (width 0.25) (layer F.Cu) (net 7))
 (segment (start 145.26 108.71) (end 145.11 108.71) (width 0.25) (layer F.Cu) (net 7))
 (segment (start 143.78 110.854315) (end 143.495685 110.57) (width 0.25) (layer F.Cu) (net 7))
 (segment (start 143.495685 110.324315) (end 143.495685 110.57) (width 0.25) (layer F.Cu) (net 7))
 (segment (start 145.11 108.71) (end 143.495685 110.324315) (width 0.25) (layer F.Cu) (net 7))
 (segment (start 134.29 109.22) (end 134.29 109.52) (width 0.25) (layer B.Cu) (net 8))
 (via (at 138.6 112.3) (size 0.8) (drill 0.4) (layers F.Cu B.Cu) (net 8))
 (segment (start 140.53 112.3) (end 140.99 111.84) (width 0.25) (layer F.Cu) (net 8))
 (segment (start 138.6 112.3) (end 140.53 112.3) (width 0.25) (layer F.Cu) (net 8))
 (segment (start 138.440684 111.574999) (end 137.085001 111.574999) (width 0.25) (layer B.Cu) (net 8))
 (segment (start 138.6 112.3) (end 138.6 111.734315) (width 0.25) (layer B.Cu) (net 8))
 (segment (start 138.6 111.734315) (end 138.440684 111.574999) (width 0.25) (layer B.Cu) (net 8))
 (segment (start 137.085001 111.279999) (end 136.800001 110.994999) (width 0.25) (layer B.Cu) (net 8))
 (segment (start 137.085001 111.574999) (end 137.085001 111.279999) (width 0.25) (layer B.Cu) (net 8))
 (segment (start 136.800001 110.994999) (end 134.295001 110.994999) (width 0.25) (layer B.Cu) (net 8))
 (segment (start 134.29 110.989998) (end 134.29 109.22) (width 0.25) (layer B.Cu) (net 8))
 (segment (start 134.295001 110.994999) (end 134.29 110.989998) (width 0.25) (layer B.Cu) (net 8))
 (via (at 137.5 104.5) (size 0.8) (drill 0.4) (layers F.Cu B.Cu) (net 9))
 (via (at 138.56 106.15) (size 0.8) (drill 0.4) (layers F.Cu B.Cu) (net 9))
 (segment (start 145.26 106.71) (end 151 106.71) (width 0.5) (layer B.Cu) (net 9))
 (segment (start 145.26 106.71) (end 151 106.71) (width 0.5) (layer F.Cu) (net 9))
 (via (at 145.26 106.71) (size 0.8) (drill 0.4) (layers F.Cu B.Cu) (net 9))
 (segment (start 139.4 109.22) (end 139.4 108.58) (width 0.25) (layer B.Cu) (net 9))
 (segment (start 138.56 106.15) (end 138.02 105.61) (width 0.25) (layer B.Cu) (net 9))
 (segment (start 134.921237 106.343763) (end 134.921237 105.808763) (width 0.25) (layer B.Cu) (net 9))
 (segment (start 134.365 106.9) (end 134.921237 106.343763) (width 0.25) (layer B.Cu) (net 9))
 (segment (start 134.921237 105.808763) (end 135.12 105.61) (width 0.25) (layer B.Cu) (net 9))
 (segment (start 139.12 106.71) (end 138.56 106.15) (width 0.25) (layer F.Cu) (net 9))
 (segment (start 145.26 106.71) (end 139.4 106.71) (width 0.25) (layer F.Cu) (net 9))
 (segment (start 139.4 106.71) (end 139.12 106.71) (width 0.25) (layer F.Cu) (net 9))
 (segment (start 139.4 107.95) (end 139.1 107.65) (width 0.25) (layer B.Cu) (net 9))
 (segment (start 139.4 109.22) (end 139.4 107.95) (width 0.25) (layer B.Cu) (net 9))
 (segment (start 139.12 106.71) (end 139.1 106.73) (width 0.25) (layer F.Cu) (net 9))
 (via (at 139.1 107.65) (size 0.8) (drill 0.4) (layers F.Cu B.Cu) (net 9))
 (segment (start 139.1 106.73) (end 139.1 107.65) (width 0.25) (layer F.Cu) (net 9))
 (segment (start 137.5 105.6) (end 137.51 105.61) (width 0.25) (layer B.Cu) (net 9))
 (segment (start 137.5 104.5) (end 137.5 105.6) (width 0.25) (layer B.Cu) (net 9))
 (segment (start 135.12 105.61) (end 137.51 105.61) (width 0.25) (layer B.Cu) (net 9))
 (segment (start 137.51 105.61) (end 138.02 105.61) (width 0.25) (layer B.Cu) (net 9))
 (via (at 142.5 104.5) (size 0.8) (drill 0.4) (layers F.Cu B.Cu) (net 3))
 (segment (start 136.7863 109.3) (end 136.0624 109.3) (width 0.25) (layer F.Cu) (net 3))
 (segment (start 138.075001 105.424999) (end 139.075001 105.424999) (width 0.25) (layer F.Cu) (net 3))
 (segment (start 137.19 109.3) (end 137.378001 109.111999) (width 0.25) (layer F.Cu) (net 3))
 (segment (start 136.0624 109.3) (end 137.19 109.3) (width 0.25) (layer F.Cu) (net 3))
 (segment (start 137.378001 109.111999) (end 137.378001 109.011999) (width 0.25) (layer F.Cu) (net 3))
 (segment (start 137.378001 109.011999) (end 137.66 108.73) (width 0.25) (layer F.Cu) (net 3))
 (segment (start 137.66 108.73) (end 137.66 105.84) (width 0.25) (layer F.Cu) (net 3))
 (segment (start 137.66 105.84) (end 138.075001 105.424999) (width 0.25) (layer F.Cu) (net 3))
 (segment (start 141.575001 105.424999) (end 142.5 104.5) (width 0.25) (layer F.Cu) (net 3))
 (segment (start 139.075001 105.424999) (end 141.575001 105.424999) (width 0.25) (layer F.Cu) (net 3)))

